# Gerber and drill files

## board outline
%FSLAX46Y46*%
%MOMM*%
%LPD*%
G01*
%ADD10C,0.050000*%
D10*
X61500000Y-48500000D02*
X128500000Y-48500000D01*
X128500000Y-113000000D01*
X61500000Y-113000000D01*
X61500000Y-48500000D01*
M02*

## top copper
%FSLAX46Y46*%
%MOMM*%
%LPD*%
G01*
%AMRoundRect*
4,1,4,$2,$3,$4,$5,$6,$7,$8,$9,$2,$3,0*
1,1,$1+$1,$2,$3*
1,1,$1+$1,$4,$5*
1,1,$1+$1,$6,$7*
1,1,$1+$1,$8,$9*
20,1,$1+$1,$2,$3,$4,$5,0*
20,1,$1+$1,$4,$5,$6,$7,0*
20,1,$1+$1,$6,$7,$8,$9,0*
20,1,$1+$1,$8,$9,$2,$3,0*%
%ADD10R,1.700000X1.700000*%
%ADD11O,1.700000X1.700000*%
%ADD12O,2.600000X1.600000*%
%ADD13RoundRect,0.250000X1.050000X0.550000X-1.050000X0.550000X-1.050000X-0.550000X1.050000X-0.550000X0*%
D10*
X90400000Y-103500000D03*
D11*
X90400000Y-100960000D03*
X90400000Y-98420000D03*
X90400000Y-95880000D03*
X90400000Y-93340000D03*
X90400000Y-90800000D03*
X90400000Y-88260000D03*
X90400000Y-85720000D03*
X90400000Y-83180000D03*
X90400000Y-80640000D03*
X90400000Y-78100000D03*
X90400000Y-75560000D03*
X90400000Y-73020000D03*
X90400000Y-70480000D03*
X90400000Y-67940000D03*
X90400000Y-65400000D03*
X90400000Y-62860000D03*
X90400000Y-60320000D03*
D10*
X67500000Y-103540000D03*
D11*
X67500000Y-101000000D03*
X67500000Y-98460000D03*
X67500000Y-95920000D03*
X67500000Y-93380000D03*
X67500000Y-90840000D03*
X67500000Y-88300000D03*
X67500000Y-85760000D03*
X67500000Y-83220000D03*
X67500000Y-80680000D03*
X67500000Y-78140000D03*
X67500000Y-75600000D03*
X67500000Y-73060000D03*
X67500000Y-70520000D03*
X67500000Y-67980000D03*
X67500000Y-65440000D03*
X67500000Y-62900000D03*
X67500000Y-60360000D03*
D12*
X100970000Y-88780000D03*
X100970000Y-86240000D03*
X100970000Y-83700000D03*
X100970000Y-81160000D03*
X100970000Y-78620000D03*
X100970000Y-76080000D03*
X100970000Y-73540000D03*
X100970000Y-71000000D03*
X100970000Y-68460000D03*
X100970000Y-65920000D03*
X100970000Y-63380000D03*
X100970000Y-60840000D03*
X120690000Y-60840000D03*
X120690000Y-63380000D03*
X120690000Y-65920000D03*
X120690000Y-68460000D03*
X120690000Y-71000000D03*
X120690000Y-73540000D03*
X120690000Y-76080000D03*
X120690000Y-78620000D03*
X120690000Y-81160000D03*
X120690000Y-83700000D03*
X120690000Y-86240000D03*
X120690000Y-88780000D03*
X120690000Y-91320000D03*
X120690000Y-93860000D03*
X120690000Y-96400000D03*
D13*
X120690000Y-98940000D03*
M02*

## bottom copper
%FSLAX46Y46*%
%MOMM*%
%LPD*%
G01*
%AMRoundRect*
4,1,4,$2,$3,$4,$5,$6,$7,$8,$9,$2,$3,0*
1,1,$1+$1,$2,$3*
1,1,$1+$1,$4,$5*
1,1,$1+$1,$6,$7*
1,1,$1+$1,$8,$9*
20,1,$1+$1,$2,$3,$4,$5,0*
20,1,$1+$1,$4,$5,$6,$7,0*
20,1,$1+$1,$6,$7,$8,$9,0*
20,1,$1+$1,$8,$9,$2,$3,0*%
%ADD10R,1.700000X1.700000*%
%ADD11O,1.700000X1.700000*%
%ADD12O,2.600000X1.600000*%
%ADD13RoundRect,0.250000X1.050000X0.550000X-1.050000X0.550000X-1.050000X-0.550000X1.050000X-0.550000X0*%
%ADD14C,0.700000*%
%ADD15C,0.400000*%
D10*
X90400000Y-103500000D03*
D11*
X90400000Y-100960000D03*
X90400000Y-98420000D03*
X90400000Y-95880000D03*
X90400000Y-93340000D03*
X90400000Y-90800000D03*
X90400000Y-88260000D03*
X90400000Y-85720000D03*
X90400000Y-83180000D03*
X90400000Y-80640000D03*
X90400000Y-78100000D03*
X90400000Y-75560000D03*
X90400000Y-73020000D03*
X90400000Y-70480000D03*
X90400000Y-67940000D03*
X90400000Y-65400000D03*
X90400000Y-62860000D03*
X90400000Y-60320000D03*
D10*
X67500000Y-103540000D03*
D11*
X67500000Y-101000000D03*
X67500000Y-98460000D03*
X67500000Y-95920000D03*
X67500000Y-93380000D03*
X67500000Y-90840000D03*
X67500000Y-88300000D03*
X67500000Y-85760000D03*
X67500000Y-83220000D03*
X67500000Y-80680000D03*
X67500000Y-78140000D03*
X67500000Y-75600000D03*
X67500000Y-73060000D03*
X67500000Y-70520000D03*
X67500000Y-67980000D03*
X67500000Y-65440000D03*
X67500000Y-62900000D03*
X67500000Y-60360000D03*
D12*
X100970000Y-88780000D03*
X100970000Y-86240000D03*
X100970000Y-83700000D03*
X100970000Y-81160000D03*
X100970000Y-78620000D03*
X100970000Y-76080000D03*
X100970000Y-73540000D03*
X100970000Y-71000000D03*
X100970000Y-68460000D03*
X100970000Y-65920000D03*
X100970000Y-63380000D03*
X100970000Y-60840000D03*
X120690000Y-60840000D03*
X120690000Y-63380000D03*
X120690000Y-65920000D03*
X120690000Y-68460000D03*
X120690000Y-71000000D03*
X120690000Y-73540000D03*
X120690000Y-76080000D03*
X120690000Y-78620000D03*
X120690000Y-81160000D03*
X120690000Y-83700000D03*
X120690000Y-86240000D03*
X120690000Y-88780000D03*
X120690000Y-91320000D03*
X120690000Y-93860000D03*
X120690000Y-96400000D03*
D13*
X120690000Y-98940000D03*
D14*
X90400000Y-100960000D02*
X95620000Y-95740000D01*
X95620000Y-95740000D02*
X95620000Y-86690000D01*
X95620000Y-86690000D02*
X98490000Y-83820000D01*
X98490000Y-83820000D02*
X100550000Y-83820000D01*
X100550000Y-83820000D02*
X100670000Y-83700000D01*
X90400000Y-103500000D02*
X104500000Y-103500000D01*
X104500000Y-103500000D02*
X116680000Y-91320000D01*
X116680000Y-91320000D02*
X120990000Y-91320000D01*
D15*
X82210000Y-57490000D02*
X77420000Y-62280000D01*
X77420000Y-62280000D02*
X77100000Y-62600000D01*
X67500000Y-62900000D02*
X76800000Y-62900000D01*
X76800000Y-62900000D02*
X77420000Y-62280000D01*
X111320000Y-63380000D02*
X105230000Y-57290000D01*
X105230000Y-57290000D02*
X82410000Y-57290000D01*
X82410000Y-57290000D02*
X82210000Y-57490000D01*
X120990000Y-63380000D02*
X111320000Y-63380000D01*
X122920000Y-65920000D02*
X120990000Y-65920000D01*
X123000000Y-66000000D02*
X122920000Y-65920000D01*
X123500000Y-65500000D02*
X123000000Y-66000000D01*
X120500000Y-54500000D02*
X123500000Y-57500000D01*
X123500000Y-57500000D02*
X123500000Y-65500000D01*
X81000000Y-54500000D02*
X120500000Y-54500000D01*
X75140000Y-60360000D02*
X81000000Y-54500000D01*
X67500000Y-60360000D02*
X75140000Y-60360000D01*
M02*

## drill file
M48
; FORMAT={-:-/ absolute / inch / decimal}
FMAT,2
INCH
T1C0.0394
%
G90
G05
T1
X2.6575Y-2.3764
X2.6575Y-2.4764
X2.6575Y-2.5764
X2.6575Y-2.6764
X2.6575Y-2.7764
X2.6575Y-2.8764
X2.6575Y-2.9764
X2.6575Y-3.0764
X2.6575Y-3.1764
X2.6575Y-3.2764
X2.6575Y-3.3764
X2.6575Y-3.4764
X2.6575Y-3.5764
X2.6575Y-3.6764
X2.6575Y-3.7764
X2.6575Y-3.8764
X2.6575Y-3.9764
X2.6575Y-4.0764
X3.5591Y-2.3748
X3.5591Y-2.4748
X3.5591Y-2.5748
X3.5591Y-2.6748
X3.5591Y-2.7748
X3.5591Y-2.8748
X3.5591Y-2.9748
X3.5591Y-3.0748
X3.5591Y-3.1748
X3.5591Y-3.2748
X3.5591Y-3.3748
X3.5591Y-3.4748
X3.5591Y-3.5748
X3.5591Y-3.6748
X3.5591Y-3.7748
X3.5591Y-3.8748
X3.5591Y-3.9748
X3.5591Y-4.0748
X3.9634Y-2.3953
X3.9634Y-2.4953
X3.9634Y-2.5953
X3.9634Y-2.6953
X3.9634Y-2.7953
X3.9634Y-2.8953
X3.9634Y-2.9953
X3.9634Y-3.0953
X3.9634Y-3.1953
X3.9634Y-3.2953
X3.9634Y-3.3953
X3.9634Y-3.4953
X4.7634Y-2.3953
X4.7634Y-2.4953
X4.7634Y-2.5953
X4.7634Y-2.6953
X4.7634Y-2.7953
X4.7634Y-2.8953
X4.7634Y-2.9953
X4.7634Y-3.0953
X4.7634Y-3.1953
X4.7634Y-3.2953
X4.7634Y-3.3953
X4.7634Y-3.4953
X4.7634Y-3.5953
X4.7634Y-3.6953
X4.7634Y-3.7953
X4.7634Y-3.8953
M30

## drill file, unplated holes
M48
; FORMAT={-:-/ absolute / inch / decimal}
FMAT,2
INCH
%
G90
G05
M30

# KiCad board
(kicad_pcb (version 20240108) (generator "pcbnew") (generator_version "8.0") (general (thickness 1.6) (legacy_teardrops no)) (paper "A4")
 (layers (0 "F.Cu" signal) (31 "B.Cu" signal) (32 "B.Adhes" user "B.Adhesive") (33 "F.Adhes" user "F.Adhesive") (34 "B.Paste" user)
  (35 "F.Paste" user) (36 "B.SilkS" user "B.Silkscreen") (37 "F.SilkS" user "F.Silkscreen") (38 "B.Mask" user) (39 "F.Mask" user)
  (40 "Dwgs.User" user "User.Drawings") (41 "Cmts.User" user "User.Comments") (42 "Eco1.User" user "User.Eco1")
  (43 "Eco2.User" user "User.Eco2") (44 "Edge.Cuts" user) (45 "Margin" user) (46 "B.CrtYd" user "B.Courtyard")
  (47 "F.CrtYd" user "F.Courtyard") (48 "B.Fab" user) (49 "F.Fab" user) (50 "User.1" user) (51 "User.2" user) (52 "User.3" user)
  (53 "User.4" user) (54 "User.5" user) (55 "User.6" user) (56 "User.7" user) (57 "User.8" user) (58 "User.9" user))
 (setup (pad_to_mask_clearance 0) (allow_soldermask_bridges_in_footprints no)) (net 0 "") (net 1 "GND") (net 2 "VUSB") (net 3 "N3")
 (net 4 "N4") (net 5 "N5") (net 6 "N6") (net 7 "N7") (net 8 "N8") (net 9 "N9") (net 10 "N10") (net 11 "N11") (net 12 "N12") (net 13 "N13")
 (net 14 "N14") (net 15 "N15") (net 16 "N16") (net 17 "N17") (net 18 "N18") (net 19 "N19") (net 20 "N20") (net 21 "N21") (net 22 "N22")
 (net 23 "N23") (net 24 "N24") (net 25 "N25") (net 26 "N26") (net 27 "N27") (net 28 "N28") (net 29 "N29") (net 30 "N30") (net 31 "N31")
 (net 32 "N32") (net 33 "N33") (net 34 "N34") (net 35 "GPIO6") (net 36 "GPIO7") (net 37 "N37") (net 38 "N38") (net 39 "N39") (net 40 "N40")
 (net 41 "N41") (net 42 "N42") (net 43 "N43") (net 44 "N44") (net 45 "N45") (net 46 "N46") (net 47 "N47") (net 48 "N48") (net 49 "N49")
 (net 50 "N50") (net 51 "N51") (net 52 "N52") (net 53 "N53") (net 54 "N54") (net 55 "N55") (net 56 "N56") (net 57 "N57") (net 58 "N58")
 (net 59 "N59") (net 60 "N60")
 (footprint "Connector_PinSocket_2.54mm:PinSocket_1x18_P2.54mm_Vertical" (layer "F.Cu") (at 90.4 103.5 180)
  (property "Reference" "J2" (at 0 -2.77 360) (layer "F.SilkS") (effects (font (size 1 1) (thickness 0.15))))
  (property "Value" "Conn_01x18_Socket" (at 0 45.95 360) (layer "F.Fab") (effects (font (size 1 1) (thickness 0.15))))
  (pad "1" thru_hole rect (at 0 0 180) (size 1.7 1.7) (drill 1) (layers "*.Cu" "*.Mask") (remove_unused_layers no) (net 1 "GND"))
  (pad "2" thru_hole oval (at 0 2.54 180) (size 1.7 1.7) (drill 1) (layers "*.Cu" "*.Mask") (remove_unused_layers no) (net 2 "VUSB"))
  (pad "3" thru_hole oval (at 0 5.08 180) (size 1.7 1.7) (drill 1) (layers "*.Cu" "*.Mask") (remove_unused_layers no) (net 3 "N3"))
  (pad "4" thru_hole oval (at 0 7.62 180) (size 1.7 1.7) (drill 1) (layers "*.Cu" "*.Mask") (remove_unused_layers no) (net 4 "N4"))
  (pad "5" thru_hole oval (at 0 10.16 180) (size 1.7 1.7) (drill 1) (layers "*.Cu" "*.Mask") (remove_unused_layers no) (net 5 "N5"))
  (pad "6" thru_hole oval (at 0 12.7 180) (size 1.7 1.7) (drill 1) (layers "*.Cu" "*.Mask") (remove_unused_layers no) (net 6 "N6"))
  (pad "7" thru_hole oval (at 0 15.24 180) (size 1.7 1.7) (drill 1) (layers "*.Cu" "*.Mask") (remove_unused_layers no) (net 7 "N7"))
  (pad "8" thru_hole oval (at 0 17.78 180) (size 1.7 1.7) (drill 1) (layers "*.Cu" "*.Mask") (remove_unused_layers no) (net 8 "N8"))
  (pad "9" thru_hole oval (at 0 20.32 180) (size 1.7 1.7) (drill 1) (layers "*.Cu" "*.Mask") (remove_unused_layers no) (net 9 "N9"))
  (pad "10" thru_hole oval (at 0 22.86 180) (size 1.7 1.7) (drill 1) (layers "*.Cu" "*.Mask") (remove_unused_layers no) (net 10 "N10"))
  (pad "11" thru_hole oval (at 0 25.4 180) (size 1.7 1.7) (drill 1) (layers "*.Cu" "*.Mask") (remove_unused_layers no) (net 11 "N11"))
  (pad "12" thru_hole oval (at 0 27.94 180) (size 1.7 1.7) (drill 1) (layers "*.Cu" "*.Mask") (remove_unused_layers no) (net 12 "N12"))
  (pad "13" thru_hole oval (at 0 30.48 180) (size 1.7 1.7) (drill 1) (layers "*.Cu" "*.Mask") (remove_unused_layers no) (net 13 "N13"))
  (pad "14" thru_hole oval (at 0 33.02 180) (size 1.7 1.7) (drill 1) (layers "*.Cu" "*.Mask") (remove_unused_layers no) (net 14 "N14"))
  (pad "15" thru_hole oval (at 0 35.56 180) (size 1.7 1.7) (drill 1) (layers "*.Cu" "*.Mask") (remove_unused_layers no) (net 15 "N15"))
  (pad "16" thru_hole oval (at 0 38.1 180) (size 1.7 1.7) (drill 1) (layers "*.Cu" "*.Mask") (remove_unused_layers no) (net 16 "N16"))
  (pad "17" thru_hole oval (at 0 40.64 180) (size 1.7 1.7) (drill 1) (layers "*.Cu" "*.Mask") (remove_unused_layers no) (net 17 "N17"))
  (pad "18" thru_hole oval (at 0 43.18 180) (size 1.7 1.7) (drill 1) (layers "*.Cu" "*.Mask") (remove_unused_layers no) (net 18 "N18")))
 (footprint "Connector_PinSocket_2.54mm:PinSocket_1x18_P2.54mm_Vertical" (layer "F.Cu") (at 67.5 103.54 180)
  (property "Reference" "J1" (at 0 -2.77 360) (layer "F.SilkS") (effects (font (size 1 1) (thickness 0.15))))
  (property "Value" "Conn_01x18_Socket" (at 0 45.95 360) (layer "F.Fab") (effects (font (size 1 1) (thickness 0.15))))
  (pad "1" thru_hole rect (at 0 0 180) (size 1.7 1.7) (drill 1) (layers "*.Cu" "*.Mask") (remove_unused_layers no) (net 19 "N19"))
  (pad "2" thru_hole oval (at 0 2.54 180) (size 1.7 1.7) (drill 1) (layers "*.Cu" "*.Mask") (remove_unused_layers no) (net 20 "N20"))
  (pad "3" thru_hole oval (at 0 5.08 180) (size 1.7 1.7) (drill 1) (layers "*.Cu" "*.Mask") (remove_unused_layers no) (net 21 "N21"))
  (pad "4" thru_hole oval (at 0 7.62 180) (size 1.7 1.7) (drill 1) (layers "*.Cu" "*.Mask") (remove_unused_layers no) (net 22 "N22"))
  (pad "5" thru_hole oval (at 0 10.16 180) (size 1.7 1.7) (drill 1) (layers "*.Cu" "*.Mask") (remove_unused_layers no) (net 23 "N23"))
  (pad "6" thru_hole oval (at 0 12.7 180) (size 1.7 1.7) (drill 1) (layers "*.Cu" "*.Mask") (remove_unused_layers no) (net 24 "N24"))
  (pad "7" thru_hole oval (at 0 15.24 180) (size 1.7 1.7) (drill 1) (layers "*.Cu" "*.Mask") (remove_unused_layers no) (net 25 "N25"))
  (pad "8" thru_hole oval (at 0 17.78 180) (size 1.7 1.7) (drill 1) (layers "*.Cu" "*.Mask") (remove_unused_layers no) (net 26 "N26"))
  (pad "9" thru_hole oval (at 0 20.32 180) (size 1.7 1.7) (drill 1) (layers "*.Cu" "*.Mask") (remove_unused_layers no) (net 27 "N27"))
  (pad "10" thru_hole oval (at 0 22.86 180) (size 1.7 1.7) (drill 1) (layers "*.Cu" "*.Mask") (remove_unused_layers no) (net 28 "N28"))
  (pad "11" thru_hole oval (at 0 25.4 180) (size 1.7 1.7) (drill 1) (layers "*.Cu" "*.Mask") (remove_unused_layers no) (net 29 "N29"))
  (pad "12" thru_hole oval (at 0 27.94 180) (size 1.7 1.7) (drill 1) (layers "*.Cu" "*.Mask") (remove_unused_layers no) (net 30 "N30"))
  (pad "13" thru_hole oval (at 0 30.48 180) (size 1.7 1.7) (drill 1) (layers "*.Cu" "*.Mask") (remove_unused_layers no) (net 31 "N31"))
  (pad "14" thru_hole oval (at 0 33.02 180) (size 1.7 1.7) (drill 1) (layers "*.Cu" "*.Mask") (remove_unused_layers no) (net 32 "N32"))
  (pad "15" thru_hole oval (at 0 35.56 180) (size 1.7 1.7) (drill 1) (layers "*.Cu" "*.Mask") (remove_unused_layers no) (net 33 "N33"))
  (pad "16" thru_hole oval (at 0 38.1 180) (size 1.7 1.7) (drill 1) (layers "*.Cu" "*.Mask") (remove_unused_layers no) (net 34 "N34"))
  (pad "17" thru_hole oval (at 0 40.64 180) (size 1.7 1.7) (drill 1) (layers "*.Cu" "*.Mask") (remove_unused_layers no) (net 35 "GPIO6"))
  (pad "18" thru_hole oval (at 0 43.18 180) (size 1.7 1.7) (drill 1) (layers "*.Cu" "*.Mask") (remove_unused_layers no) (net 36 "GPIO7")))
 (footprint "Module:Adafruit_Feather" (layer "F.Cu") (at 120.99 98.94 180)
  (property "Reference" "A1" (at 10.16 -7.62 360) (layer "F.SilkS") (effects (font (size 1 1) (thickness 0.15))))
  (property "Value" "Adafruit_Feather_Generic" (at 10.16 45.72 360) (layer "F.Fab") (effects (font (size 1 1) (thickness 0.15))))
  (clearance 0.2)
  (pad "1" thru_hole roundrect (at 0 0 180) (size 2.6 1.6) (drill 1 (offset 0.3 0)) (layers "*.Cu" "*.Mask") (remove_unused_layers no)
   (roundrect_rratio 0.15625) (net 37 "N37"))
  (pad "2" thru_hole oval (at 0 2.54 180) (size 2.6 1.6) (drill 1 (offset 0.3 0)) (layers "*.Cu" "*.Mask") (remove_unused_layers no)
   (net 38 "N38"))
  (pad "3" thru_hole oval (at 0 5.08 180) (size 2.6 1.6) (drill 1 (offset 0.3 0)) (layers "*.Cu" "*.Mask") (remove_unused_layers no)
   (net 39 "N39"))
  (pad "4" thru_hole oval (at 0 7.62 180) (size 2.6 1.6) (drill 1 (offset 0.3 0)) (layers "*.Cu" "*.Mask") (remove_unused_layers no)
   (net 1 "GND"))
  (pad "5" thru_hole oval (at 0 10.16 180) (size 2.6 1.6) (drill 1 (offset 0.3 0)) (layers "*.Cu" "*.Mask") (remove_unused_layers no)
   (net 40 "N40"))
  (pad "6" thru_hole oval (at 0 12.7 180) (size 2.6 1.6) (drill 1 (offset 0.3 0)) (layers "*.Cu" "*.Mask") (remove_unused_layers no)
   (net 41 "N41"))
  (pad "7" thru_hole oval (at 0 15.24 180) (size 2.6 1.6) (drill 1 (offset 0.3 0)) (layers "*.Cu" "*.Mask") (remove_unused_layers no)
   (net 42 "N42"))
  (pad "8" thru_hole oval (at 0 17.78 180) (size 2.6 1.6) (drill 1 (offset 0.3 0)) (layers "*.Cu" "*.Mask") (remove_unused_layers no)
   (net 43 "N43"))
  (pad "9" thru_hole oval (at 0 20.32 180) (size 2.6 1.6) (drill 1 (offset 0.3 0)) (layers "*.Cu" "*.Mask") (remove_unused_layers no)
   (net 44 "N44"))
  (pad "10" thru_hole oval (at 0 22.86 180) (size 2.6 1.6) (drill 1 (offset 0.3 0)) (layers "*.Cu" "*.Mask") (remove_unused_layers no)
   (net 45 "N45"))
  (pad "11" thru_hole oval (at 0 25.4 180) (size 2.6 1.6) (drill 1 (offset 0.3 0)) (layers "*.Cu" "*.Mask") (remove_unused_layers no)
   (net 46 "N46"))
  (pad "12" thru_hole oval (at 0 27.94 180) (size 2.6 1.6) (drill 1 (offset 0.3 0)) (layers "*.Cu" "*.Mask") (remove_unused_layers no)
   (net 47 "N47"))
  (pad "13" thru_hole oval (at 0 30.48 180) (size 2.6 1.6) (drill 1 (offset 0.3 0)) (layers "*.Cu" "*.Mask") (remove_unused_layers no)
   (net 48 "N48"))
  (pad "14" thru_hole oval (at 0 33.02 180) (size 2.6 1.6) (drill 1 (offset 0.3 0)) (layers "*.Cu" "*.Mask") (remove_unused_layers no)
   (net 36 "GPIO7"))
  (pad "15" thru_hole oval (at 0 35.56 180) (size 2.6 1.6) (drill 1 (offset 0.3 0)) (layers "*.Cu" "*.Mask") (remove_unused_layers no)
   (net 35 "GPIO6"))
  (pad "16" thru_hole oval (at 0 38.1 180) (size 2.6 1.6) (drill 1 (offset 0.3 0)) (layers "*.Cu" "*.Mask") (remove_unused_layers no)
   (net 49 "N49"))
  (pad "17" thru_hole oval (at 20.32 38.1) (size 2.6 1.6) (drill 1 (offset 0.3 0)) (layers "*.Cu" "*.Mask") (remove_unused_layers no)
   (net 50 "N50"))
  (pad "18" thru_hole oval (at 20.32 35.56) (size 2.6 1.6) (drill 1 (offset 0.3 0)) (layers "*.Cu" "*.Mask") (remove_unused_layers no)
   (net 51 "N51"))
  (pad "19" thru_hole oval (at 20.32 33.02) (size 2.6 1.6) (drill 1 (offset 0.3 0)) (layers "*.Cu" "*.Mask") (remove_unused_layers no)
   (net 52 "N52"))
  (pad "20" thru_hole oval (at 20.32 30.48) (size 2.6 1.6) (drill 1 (offset 0.3 0)) (layers "*.Cu" "*.Mask") (remove_unused_layers no)
   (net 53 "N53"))
  (pad "21" thru_hole oval (at 20.32 27.94) (size 2.6 1.6) (drill 1 (offset 0.3 0)) (layers "*.Cu" "*.Mask") (remove_unused_layers no)
   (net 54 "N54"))
  (pad "22" thru_hole oval (at 20.32 25.4) (size 2.6 1.6) (drill 1 (offset 0.3 0)) (layers "*.Cu" "*.Mask") (remove_unused_layers no)
   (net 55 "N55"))
  (pad "23" thru_hole oval (at 20.32 22.86) (size 2.6 1.6) (drill 1 (offset 0.3 0)) (layers "*.Cu" "*.Mask") (remove_unused_layers no)
   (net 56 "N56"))
  (pad "24" thru_hole oval (at 20.32 20.32) (size 2.6 1.6) (drill 1 (offset 0.3 0)) (layers "*.Cu" "*.Mask") (remove_unused_layers no)
   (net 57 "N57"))
  (pad "25" thru_hole oval (at 20.32 17.78) (size 2.6 1.6) (drill 1 (offset 0.3 0)) (layers "*.Cu" "*.Mask") (remove_unused_layers no)
   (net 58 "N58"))
  (pad "26" thru_hole oval (at 20.32 15.24) (size 2.6 1.6) (drill 1 (offset 0.3 0)) (layers "*.Cu" "*.Mask") (remove_unused_layers no)
   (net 2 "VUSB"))
  (pad "27" thru_hole oval (at 20.32 12.7) (size 2.6 1.6) (drill 1 (offset 0.3 0)) (layers "*.Cu" "*.Mask") (remove_unused_layers no)
   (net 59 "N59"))
  (pad "28" thru_hole oval (at 20.32 10.16) (size 2.6 1.6) (drill 1 (offset 0.3 0)) (layers "*.Cu" "*.Mask") (remove_unused_layers no)
   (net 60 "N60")))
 (gr_rect (start 61.5 48.5) (end 128.5 113) (stroke (width 0.05) (type default)) (fill none) (layer "Edge.Cuts"))
 (segment (start 98.49 83.82) (end 100.55 83.82) (width 0.7) (layer "B.Cu") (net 2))
 (segment (start 95.62 95.74) (end 95.62 86.69) (width 0.7) (layer "B.Cu") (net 2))
 (segment (start 100.55 83.82) (end 100.67 83.7) (width 0.7) (layer "B.Cu") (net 2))
 (segment (start 95.62 86.69) (end 98.49 83.82) (width 0.7) (layer "B.Cu") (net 2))
 (segment (start 90.4 100.96) (end 95.62 95.74) (width 0.7) (layer "B.Cu") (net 2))
 (segment (start 67.5 60.36) (end 75.14 60.36) (width 0.4) (layer "B.Cu") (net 36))
 (segment (start 120.5 54.5) (end 123.5 57.5) (width 0.4) (layer "B.Cu") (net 36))
 (segment (start 81 54.5) (end 120.5 54.5) (width 0.4) (layer "B.Cu") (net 36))
 (segment (start 75.14 60.36) (end 81 54.5) (width 0.4) (layer "B.Cu") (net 36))
 (segment (start 123.5 57.5) (end 123.5 65.5) (width 0.4) (layer "B.Cu") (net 36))
 (segment (start 123 66) (end 122.92 65.92) (width 0.4) (layer "B.Cu") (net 36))
 (segment (start 123.5 65.5) (end 123 66) (width 0.4) (layer "B.Cu") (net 36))
 (segment (start 122.92 65.92) (end 120.99 65.92) (width 0.4) (layer "B.Cu") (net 36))
 (segment (start 82.21 57.49) (end 77.42 62.28) (width 0.4) (layer "B.Cu") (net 35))
 (segment (start 77.42 62.28) (end 77.1 62.6) (width 0.4) (layer "B.Cu") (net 35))
 (segment (start 67.5 62.9) (end 76.8 62.9) (width 0.4) (layer "B.Cu") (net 35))
 (segment (start 120.99 63.38) (end 111.32 63.38) (width 0.4) (layer "B.Cu") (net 35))
 (segment (start 76.8 62.9) (end 77.42 62.28) (width 0.4) (layer "B.Cu") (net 35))
 (segment (start 105.23 57.29) (end 82.41 57.29) (width 0.4) (layer "B.Cu") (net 35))
 (segment (start 82.41 57.29) (end 82.21 57.49) (width 0.4) (layer "B.Cu") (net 35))
 (segment (start 111.32 63.38) (end 105.23 57.29) (width 0.4) (layer "B.Cu") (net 35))
 (segment (start 104.5 103.5) (end 116.68 91.32) (width 0.7) (layer "B.Cu") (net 1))
 (segment (start 116.68 91.32) (end 120.99 91.32) (width 0.7) (layer "B.Cu") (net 1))
 (segment (start 90.4 103.5) (end 104.5 103.5) (width 0.7) (layer "B.Cu") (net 1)))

